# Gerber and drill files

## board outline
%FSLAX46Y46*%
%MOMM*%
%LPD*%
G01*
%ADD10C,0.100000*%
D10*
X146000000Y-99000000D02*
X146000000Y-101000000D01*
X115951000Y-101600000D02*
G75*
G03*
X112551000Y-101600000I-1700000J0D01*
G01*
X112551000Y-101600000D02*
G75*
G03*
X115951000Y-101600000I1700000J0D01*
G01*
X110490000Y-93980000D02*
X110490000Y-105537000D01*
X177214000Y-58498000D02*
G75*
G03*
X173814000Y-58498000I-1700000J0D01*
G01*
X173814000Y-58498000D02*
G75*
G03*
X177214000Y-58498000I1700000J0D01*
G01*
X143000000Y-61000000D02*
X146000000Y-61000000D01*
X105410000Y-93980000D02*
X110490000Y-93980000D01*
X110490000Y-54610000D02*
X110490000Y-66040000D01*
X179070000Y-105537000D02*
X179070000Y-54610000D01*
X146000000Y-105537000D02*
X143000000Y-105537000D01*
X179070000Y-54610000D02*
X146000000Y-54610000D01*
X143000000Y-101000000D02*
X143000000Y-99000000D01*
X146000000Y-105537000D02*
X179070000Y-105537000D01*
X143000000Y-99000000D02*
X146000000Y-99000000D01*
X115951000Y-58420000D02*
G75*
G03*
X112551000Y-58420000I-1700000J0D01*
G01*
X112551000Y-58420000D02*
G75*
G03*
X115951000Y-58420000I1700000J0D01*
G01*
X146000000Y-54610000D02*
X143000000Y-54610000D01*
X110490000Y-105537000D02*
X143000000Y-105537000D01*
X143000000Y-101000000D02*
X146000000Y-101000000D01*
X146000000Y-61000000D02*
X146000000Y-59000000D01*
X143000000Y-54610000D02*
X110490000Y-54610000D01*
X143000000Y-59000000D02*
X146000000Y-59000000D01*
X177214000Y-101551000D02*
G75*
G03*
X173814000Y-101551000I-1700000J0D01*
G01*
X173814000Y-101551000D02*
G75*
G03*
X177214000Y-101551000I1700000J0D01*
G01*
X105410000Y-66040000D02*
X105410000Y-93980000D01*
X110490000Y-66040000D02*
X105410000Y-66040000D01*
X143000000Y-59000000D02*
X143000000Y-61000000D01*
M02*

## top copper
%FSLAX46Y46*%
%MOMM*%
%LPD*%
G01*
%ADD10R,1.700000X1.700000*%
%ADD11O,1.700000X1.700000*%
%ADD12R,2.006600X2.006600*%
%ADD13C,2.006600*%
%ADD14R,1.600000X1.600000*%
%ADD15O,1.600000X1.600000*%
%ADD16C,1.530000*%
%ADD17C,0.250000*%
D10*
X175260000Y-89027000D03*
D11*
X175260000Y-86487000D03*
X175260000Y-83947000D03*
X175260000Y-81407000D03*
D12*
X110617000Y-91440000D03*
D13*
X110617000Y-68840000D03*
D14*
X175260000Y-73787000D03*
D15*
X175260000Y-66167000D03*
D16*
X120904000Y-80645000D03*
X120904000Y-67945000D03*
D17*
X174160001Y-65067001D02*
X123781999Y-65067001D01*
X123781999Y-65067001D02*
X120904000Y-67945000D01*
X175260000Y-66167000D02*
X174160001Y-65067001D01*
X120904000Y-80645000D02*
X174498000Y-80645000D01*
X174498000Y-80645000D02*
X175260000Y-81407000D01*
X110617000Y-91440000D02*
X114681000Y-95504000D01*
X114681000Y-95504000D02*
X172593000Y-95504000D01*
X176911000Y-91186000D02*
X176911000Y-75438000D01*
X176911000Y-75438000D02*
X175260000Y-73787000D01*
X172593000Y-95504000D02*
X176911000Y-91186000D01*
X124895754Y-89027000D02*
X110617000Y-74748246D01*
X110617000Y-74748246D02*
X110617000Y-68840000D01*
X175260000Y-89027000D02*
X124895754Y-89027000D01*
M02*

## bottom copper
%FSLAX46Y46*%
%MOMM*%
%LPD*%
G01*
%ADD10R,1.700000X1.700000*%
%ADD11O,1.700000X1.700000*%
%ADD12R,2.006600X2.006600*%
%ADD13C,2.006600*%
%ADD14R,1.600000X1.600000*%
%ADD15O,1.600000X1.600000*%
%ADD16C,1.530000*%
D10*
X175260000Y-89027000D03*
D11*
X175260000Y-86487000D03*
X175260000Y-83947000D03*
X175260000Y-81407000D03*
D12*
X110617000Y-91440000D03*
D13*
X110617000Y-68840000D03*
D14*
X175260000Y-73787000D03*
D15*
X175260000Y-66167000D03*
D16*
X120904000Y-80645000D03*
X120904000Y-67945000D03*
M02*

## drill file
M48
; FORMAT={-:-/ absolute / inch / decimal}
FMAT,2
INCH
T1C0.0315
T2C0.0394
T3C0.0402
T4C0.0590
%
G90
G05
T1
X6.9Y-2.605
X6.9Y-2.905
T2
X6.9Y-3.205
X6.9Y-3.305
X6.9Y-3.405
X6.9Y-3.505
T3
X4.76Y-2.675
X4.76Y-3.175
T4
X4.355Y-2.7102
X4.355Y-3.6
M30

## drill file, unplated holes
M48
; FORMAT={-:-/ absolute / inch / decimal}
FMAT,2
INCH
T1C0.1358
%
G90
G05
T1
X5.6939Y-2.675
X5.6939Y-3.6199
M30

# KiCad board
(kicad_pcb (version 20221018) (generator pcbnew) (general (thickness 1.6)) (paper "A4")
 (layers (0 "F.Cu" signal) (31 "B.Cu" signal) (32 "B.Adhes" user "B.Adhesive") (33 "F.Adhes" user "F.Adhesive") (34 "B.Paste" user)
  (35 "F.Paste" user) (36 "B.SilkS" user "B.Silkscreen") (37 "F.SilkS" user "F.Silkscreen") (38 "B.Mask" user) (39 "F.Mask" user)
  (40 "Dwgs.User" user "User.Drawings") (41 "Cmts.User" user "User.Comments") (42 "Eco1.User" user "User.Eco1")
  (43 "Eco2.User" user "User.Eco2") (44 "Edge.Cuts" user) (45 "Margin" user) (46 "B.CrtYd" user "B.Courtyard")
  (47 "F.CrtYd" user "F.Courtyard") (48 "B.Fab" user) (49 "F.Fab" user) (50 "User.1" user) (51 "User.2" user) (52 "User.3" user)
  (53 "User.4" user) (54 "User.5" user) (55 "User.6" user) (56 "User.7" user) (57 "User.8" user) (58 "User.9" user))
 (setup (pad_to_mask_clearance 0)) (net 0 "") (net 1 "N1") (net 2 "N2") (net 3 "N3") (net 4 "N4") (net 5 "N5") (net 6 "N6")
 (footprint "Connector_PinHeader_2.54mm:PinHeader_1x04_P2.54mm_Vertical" (layer "F.Cu") (at 175.26 89.027 180)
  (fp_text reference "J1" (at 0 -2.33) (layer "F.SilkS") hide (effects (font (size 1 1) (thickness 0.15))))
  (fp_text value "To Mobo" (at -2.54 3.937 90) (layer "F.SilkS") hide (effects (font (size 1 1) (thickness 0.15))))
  (pad "1" thru_hole rect (at 0 0 180) (size 1.7 1.7) (drill 1) (layers "*.Cu" "*.Mask") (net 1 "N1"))
  (pad "2" thru_hole oval (at 0 2.54 180) (size 1.7 1.7) (drill 1) (layers "*.Cu" "*.Mask") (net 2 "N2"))
  (pad "3" thru_hole oval (at 0 5.08 180) (size 1.7 1.7) (drill 1) (layers "*.Cu" "*.Mask") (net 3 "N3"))
  (pad "4" thru_hole oval (at 0 7.62 180) (size 1.7 1.7) (drill 1) (layers "*.Cu" "*.Mask") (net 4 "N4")))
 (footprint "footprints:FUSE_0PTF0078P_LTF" (layer "F.Cu") (at 110.617 91.44 90)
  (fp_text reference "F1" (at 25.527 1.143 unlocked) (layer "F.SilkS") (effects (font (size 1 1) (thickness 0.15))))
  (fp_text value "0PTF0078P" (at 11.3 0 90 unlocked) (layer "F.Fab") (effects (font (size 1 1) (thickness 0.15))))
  (pad "1" thru_hole rect (at 0 0 90) (size 2.0066 2.0066) (drill 1.4986) (layers "*.Cu" "*.Mask") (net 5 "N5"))
  (pad "2" thru_hole circle (at 22.6 0 90) (size 2.0066 2.0066) (drill 1.4986) (layers "*.Cu" "*.Mask") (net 1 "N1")))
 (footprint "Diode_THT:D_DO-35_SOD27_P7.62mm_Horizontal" (layer "F.Cu") (at 175.26 73.787 90)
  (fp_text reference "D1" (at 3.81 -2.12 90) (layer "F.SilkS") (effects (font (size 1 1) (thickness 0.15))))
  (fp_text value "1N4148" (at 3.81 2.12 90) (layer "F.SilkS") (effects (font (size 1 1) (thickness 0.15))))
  (pad "1" thru_hole rect (at 0 0 90) (size 1.6 1.6) (drill 0.8) (layers "*.Cu" "*.Mask") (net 5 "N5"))
  (pad "2" thru_hole oval (at 7.62 0 90) (size 1.6 1.6) (drill 0.8) (layers "*.Cu" "*.Mask") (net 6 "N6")))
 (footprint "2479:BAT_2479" (layer "F.Cu") (at 144.624 79.945 180)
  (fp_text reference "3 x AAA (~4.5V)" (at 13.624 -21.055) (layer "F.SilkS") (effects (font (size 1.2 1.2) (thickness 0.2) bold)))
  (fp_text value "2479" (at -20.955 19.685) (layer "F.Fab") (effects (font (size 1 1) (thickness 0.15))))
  (pad "" np_thru_hole circle (at 0 -12 180) (size 3.45 3.45) (drill 3.45) (layers "*.Cu" "*.Mask"))
  (pad "" np_thru_hole circle (at 0 12 180) (size 3.45 3.45) (drill 3.45) (layers "*.Cu" "*.Mask"))
  (pad "N" thru_hole circle (at 23.72 -0.7 180) (size 1.53 1.53) (drill 1.02) (layers "*.Cu" "*.Mask") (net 4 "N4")
   (solder_mask_margin 0.102))
  (pad "P" thru_hole circle (at 23.72 12 180) (size 1.53 1.53) (drill 1.02) (layers "*.Cu" "*.Mask") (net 6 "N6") (solder_mask_margin 0.102)))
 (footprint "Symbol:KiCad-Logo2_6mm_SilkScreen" (layer "B.Cu") (at 122 72 180)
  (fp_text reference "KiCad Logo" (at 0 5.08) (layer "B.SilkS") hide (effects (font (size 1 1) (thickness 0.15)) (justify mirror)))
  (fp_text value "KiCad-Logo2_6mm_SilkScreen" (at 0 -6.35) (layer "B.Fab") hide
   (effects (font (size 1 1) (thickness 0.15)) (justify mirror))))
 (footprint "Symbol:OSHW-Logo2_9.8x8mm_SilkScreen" (layer "B.Cu") (at 111 83 180)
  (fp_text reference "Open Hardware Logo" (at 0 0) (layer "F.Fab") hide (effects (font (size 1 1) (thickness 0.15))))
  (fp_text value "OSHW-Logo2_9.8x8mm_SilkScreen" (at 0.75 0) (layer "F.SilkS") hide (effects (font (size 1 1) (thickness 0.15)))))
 (gr_line (start 146 99) (end 146 101) (stroke (width 0.1) (type default)) (layer "Edge.Cuts"))
 (gr_circle (center 114.251 101.6) (end 115.951 101.6) (stroke (width 0.1) (type default)) (fill none) (layer "Edge.Cuts"))
 (gr_line (start 110.49 93.98) (end 110.49 105.537) (stroke (width 0.1) (type default)) (layer "Edge.Cuts"))
 (gr_circle (center 175.514 58.498) (end 177.214 58.498) (stroke (width 0.1) (type default)) (fill none) (layer "Edge.Cuts"))
 (gr_line (start 143 61) (end 146 61) (stroke (width 0.1) (type default)) (layer "Edge.Cuts"))
 (gr_line (start 105.41 93.98) (end 110.49 93.98) (stroke (width 0.1) (type default)) (layer "Edge.Cuts"))
 (gr_line (start 110.49 54.61) (end 110.49 66.04) (stroke (width 0.1) (type default)) (layer "Edge.Cuts"))
 (gr_line (start 179.07 105.537) (end 179.07 54.61) (stroke (width 0.1) (type default)) (layer "Edge.Cuts"))
 (gr_line (start 146 105.537) (end 143 105.537) (stroke (width 0.1) (type default)) (layer "Edge.Cuts"))
 (gr_line (start 179.07 54.61) (end 146 54.61) (stroke (width 0.1) (type default)) (layer "Edge.Cuts"))
 (gr_line (start 143 101) (end 143 99) (stroke (width 0.1) (type default)) (layer "Edge.Cuts"))
 (gr_line (start 146 105.537) (end 179.07 105.537) (stroke (width 0.1) (type default)) (layer "Edge.Cuts"))
 (gr_line (start 143 99) (end 146 99) (stroke (width 0.1) (type default)) (layer "Edge.Cuts"))
 (gr_circle (center 114.251 58.42) (end 115.951 58.42) (stroke (width 0.1) (type default)) (fill none) (layer "Edge.Cuts"))
 (gr_line (start 146 54.61) (end 143 54.61) (stroke (width 0.1) (type default)) (layer "Edge.Cuts"))
 (gr_line (start 110.49 105.537) (end 143 105.537) (stroke (width 0.1) (type default)) (layer "Edge.Cuts"))
 (gr_line (start 143 101) (end 146 101) (stroke (width 0.1) (type default)) (layer "Edge.Cuts"))
 (gr_line (start 146 61) (end 146 59) (stroke (width 0.1) (type default)) (layer "Edge.Cuts"))
 (gr_line (start 143 54.61) (end 110.49 54.61) (stroke (width 0.1) (type default)) (layer "Edge.Cuts"))
 (gr_line (start 143 59) (end 146 59) (stroke (width 0.1) (type default)) (layer "Edge.Cuts"))
 (gr_circle (center 175.514 101.551) (end 177.214 101.551) (stroke (width 0.1) (type default)) (fill none) (layer "Edge.Cuts"))
 (gr_line (start 105.41 66.04) (end 105.41 93.98) (stroke (width 0.1) (type default)) (layer "Edge.Cuts"))
 (gr_line (start 110.49 66.04) (end 105.41 66.04) (stroke (width 0.1) (type default)) (layer "Edge.Cuts"))
 (gr_line (start 143 59) (end 143 61) (stroke (width 0.1) (type default)) (layer "Edge.Cuts"))
 (segment (start 174.160001 65.067001) (end 123.781999 65.067001) (width 0.25) (layer "F.Cu") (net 6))
 (segment (start 123.781999 65.067001) (end 120.904 67.945) (width 0.25) (layer "F.Cu") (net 6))
 (segment (start 175.26 66.167) (end 174.160001 65.067001) (width 0.25) (layer "F.Cu") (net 6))
 (segment (start 120.904 80.645) (end 174.498 80.645) (width 0.25) (layer "F.Cu") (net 4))
 (segment (start 174.498 80.645) (end 175.26 81.407) (width 0.25) (layer "F.Cu") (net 4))
 (segment (start 110.617 91.44) (end 114.681 95.504) (width 0.25) (layer "F.Cu") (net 5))
 (segment (start 114.681 95.504) (end 172.593 95.504) (width 0.25) (layer "F.Cu") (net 5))
 (segment (start 176.911 91.186) (end 176.911 75.438) (width 0.25) (layer "F.Cu") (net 5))
 (segment (start 176.911 75.438) (end 175.26 73.787) (width 0.25) (layer "F.Cu") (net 5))
 (segment (start 172.593 95.504) (end 176.911 91.186) (width 0.25) (layer "F.Cu") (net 5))
 (segment (start 124.895754 89.027) (end 110.617 74.748246) (width 0.25) (layer "F.Cu") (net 1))
 (segment (start 110.617 74.748246) (end 110.617 68.84) (width 0.25) (layer "F.Cu") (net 1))
 (segment (start 175.26 89.027) (end 124.895754 89.027) (width 0.25) (layer "F.Cu") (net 1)))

